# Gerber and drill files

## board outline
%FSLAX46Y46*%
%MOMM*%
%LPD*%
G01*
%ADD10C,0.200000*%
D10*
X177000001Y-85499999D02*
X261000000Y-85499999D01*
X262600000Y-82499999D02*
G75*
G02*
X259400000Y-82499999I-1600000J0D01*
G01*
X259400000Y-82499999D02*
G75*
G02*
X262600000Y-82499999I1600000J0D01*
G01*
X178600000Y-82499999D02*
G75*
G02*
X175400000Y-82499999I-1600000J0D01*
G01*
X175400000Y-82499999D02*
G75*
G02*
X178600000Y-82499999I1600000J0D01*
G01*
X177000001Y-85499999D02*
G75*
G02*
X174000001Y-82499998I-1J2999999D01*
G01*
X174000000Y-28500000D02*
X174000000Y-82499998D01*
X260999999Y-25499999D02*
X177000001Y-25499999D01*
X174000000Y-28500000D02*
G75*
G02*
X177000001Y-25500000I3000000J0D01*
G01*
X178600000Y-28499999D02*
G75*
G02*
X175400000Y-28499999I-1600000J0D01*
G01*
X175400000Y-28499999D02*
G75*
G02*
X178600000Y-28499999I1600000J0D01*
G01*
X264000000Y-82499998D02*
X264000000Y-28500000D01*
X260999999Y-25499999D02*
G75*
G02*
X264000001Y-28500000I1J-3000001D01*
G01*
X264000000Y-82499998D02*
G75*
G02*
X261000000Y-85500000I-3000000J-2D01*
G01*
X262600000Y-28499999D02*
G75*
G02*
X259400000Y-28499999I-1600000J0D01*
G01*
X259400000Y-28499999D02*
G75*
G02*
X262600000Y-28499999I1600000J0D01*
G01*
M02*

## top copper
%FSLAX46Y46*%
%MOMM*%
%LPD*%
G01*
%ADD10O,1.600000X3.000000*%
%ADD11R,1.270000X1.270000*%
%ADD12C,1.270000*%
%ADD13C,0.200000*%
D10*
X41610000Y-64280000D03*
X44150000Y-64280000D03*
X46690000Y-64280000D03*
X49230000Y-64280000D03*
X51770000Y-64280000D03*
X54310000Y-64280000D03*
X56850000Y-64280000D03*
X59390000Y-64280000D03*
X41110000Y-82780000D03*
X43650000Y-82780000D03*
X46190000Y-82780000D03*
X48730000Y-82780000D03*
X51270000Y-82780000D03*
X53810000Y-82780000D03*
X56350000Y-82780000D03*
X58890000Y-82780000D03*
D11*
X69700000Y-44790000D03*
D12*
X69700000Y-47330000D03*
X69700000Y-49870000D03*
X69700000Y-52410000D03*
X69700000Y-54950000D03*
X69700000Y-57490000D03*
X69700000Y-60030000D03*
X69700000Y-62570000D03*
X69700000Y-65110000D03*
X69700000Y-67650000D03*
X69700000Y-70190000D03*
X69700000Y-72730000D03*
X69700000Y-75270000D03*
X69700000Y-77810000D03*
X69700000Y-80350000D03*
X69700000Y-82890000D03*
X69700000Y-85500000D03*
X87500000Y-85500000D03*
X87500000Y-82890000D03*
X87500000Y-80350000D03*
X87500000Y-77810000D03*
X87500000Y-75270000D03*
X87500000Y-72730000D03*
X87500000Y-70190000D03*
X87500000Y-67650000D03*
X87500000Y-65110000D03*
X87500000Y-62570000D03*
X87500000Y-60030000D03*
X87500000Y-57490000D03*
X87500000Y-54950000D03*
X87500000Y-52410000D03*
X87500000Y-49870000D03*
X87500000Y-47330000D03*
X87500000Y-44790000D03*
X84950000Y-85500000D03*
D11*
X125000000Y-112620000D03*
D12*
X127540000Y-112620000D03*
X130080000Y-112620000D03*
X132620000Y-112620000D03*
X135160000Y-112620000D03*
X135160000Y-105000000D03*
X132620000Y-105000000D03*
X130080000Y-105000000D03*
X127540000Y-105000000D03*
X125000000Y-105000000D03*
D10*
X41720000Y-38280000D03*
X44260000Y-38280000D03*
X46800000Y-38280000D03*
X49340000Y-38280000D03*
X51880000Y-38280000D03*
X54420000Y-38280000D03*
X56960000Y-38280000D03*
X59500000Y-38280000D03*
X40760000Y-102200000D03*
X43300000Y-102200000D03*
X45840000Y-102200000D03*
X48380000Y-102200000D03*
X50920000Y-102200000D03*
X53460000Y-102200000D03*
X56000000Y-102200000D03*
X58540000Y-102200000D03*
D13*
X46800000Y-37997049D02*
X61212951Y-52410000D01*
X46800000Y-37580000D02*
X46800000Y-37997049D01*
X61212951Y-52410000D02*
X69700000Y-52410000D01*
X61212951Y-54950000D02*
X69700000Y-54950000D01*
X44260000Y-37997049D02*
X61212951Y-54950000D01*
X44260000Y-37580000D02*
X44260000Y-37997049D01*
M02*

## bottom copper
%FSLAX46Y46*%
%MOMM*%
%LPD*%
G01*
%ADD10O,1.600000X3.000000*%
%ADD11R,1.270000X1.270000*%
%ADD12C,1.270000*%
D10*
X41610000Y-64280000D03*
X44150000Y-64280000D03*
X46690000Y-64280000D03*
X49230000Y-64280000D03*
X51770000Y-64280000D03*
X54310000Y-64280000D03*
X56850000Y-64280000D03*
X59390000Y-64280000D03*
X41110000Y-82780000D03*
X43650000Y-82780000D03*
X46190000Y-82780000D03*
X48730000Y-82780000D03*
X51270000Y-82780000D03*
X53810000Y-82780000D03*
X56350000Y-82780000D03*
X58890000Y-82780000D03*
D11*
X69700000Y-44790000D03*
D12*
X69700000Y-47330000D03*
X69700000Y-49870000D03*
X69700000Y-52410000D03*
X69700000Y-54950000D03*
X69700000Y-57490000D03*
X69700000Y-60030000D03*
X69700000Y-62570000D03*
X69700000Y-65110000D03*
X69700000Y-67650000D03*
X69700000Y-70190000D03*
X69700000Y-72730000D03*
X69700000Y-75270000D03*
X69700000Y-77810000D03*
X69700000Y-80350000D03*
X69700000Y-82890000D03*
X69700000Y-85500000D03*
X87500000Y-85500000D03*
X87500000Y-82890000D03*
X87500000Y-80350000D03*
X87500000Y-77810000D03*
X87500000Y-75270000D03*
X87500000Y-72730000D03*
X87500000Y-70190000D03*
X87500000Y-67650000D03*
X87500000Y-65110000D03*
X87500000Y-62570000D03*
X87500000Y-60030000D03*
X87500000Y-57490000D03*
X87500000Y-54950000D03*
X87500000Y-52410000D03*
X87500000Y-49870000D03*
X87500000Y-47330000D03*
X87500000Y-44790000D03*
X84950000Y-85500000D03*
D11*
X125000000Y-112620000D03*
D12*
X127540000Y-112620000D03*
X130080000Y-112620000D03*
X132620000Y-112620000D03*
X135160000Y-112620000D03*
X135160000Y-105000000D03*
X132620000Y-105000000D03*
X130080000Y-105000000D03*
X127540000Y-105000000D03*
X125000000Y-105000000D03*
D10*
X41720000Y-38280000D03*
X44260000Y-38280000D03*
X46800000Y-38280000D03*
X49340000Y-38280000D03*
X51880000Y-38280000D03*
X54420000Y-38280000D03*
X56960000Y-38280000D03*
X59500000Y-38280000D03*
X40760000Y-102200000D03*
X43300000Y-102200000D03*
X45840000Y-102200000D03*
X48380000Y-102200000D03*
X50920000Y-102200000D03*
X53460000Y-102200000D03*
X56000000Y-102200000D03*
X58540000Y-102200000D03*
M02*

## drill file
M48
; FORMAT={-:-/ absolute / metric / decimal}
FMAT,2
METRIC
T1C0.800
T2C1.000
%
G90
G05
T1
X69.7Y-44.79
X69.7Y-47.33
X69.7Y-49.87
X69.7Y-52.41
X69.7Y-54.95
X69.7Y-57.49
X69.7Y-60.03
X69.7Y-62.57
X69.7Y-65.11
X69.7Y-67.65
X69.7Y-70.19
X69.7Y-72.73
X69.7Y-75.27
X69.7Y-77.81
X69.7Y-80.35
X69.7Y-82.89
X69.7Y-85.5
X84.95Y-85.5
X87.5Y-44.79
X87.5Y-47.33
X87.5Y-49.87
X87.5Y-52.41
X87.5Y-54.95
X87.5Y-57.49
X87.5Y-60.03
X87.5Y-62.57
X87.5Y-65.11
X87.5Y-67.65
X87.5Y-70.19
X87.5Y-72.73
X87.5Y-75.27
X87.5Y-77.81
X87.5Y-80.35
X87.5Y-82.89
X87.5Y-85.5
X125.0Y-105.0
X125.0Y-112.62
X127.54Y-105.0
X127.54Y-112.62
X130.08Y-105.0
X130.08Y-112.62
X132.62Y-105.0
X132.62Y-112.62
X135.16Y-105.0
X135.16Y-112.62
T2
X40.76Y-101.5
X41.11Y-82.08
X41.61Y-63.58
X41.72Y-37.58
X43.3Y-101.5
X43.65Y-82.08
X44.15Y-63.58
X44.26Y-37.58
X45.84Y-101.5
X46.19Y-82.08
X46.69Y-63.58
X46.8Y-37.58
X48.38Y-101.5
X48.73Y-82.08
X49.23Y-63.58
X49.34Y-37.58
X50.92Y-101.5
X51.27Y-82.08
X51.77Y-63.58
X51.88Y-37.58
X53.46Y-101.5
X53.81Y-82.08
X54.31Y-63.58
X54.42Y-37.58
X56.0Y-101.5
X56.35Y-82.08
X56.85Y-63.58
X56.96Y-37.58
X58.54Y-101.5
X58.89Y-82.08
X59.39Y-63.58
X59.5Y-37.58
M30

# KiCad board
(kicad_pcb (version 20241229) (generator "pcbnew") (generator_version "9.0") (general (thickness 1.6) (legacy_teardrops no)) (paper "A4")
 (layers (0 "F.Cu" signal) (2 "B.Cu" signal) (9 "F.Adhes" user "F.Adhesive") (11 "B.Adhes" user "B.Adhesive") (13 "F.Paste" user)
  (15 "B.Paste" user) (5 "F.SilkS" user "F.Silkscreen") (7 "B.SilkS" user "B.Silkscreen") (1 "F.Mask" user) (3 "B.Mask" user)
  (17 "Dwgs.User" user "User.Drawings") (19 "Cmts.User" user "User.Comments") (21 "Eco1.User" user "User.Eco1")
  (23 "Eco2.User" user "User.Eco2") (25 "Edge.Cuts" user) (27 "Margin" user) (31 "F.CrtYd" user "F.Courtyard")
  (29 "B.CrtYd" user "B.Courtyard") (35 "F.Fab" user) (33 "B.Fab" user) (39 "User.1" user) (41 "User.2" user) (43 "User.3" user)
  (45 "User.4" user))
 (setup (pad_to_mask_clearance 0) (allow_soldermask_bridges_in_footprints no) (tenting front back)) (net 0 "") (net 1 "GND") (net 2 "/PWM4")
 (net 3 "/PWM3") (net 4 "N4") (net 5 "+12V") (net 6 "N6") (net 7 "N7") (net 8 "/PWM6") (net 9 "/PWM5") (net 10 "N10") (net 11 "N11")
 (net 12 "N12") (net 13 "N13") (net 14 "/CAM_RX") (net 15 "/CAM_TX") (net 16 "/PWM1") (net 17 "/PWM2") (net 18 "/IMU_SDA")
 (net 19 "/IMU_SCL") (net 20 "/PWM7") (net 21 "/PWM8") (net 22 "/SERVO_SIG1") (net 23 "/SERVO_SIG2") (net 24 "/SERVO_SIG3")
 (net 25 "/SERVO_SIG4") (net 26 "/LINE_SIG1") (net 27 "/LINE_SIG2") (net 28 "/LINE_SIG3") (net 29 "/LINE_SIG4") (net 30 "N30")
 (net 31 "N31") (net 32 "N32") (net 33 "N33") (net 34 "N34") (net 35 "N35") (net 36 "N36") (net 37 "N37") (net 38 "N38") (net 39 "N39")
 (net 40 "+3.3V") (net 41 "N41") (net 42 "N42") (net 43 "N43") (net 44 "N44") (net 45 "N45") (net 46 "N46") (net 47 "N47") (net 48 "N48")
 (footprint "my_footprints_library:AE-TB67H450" (layer "F.Cu") (at 50.5 61.5)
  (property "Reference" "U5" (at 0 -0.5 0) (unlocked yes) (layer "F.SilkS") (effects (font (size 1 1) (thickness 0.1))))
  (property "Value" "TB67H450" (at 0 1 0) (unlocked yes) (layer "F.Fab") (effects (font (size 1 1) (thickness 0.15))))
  (pad "1" thru_hole oval (at -8.89 2.08) (size 1.6 3) (drill 1 (offset 0 0.7)) (layers "*.Cu" "*.Mask") (remove_unused_layers no)
   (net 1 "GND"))
  (pad "2" thru_hole oval (at -6.35 2.08) (size 1.6 3) (drill 1 (offset 0 0.7)) (layers "*.Cu" "*.Mask") (remove_unused_layers no)
   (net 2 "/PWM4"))
  (pad "3" thru_hole oval (at -3.81 2.08) (size 1.6 3) (drill 1 (offset 0 0.7)) (layers "*.Cu" "*.Mask") (remove_unused_layers no)
   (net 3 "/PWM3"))
  (pad "4" thru_hole oval (at -1.27 2.08) (size 1.6 3) (drill 1 (offset 0 0.7)) (layers "*.Cu" "*.Mask") (remove_unused_layers no)
   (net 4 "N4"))
  (pad "5" thru_hole oval (at 1.27 2.08) (size 1.6 3) (drill 1 (offset 0 0.7)) (layers "*.Cu" "*.Mask") (remove_unused_layers no)
   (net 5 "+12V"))
  (pad "6" thru_hole oval (at 3.81 2.08) (size 1.6 3) (drill 1 (offset 0 0.7)) (layers "*.Cu" "*.Mask") (remove_unused_layers no)
   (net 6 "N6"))
  (pad "7" thru_hole oval (at 6.35 2.08) (size 1.6 3) (drill 1 (offset 0 0.7)) (layers "*.Cu" "*.Mask") (remove_unused_layers no)
   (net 1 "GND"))
  (pad "8" thru_hole oval (at 8.89 2.08) (size 1.6 3) (drill 1 (offset 0 0.7)) (layers "*.Cu" "*.Mask") (remove_unused_layers no)
   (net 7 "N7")))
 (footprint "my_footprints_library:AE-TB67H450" (layer "F.Cu") (at 50 80)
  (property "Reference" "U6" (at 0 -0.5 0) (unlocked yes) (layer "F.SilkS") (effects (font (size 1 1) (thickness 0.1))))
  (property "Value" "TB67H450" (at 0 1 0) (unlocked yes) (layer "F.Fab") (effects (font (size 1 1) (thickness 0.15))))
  (pad "1" thru_hole oval (at -8.89 2.08) (size 1.6 3) (drill 1 (offset 0 0.7)) (layers "*.Cu" "*.Mask") (remove_unused_layers no)
   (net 1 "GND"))
  (pad "2" thru_hole oval (at -6.35 2.08) (size 1.6 3) (drill 1 (offset 0 0.7)) (layers "*.Cu" "*.Mask") (remove_unused_layers no)
   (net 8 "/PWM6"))
  (pad "3" thru_hole oval (at -3.81 2.08) (size 1.6 3) (drill 1 (offset 0 0.7)) (layers "*.Cu" "*.Mask") (remove_unused_layers no)
   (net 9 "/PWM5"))
  (pad "4" thru_hole oval (at -1.27 2.08) (size 1.6 3) (drill 1 (offset 0 0.7)) (layers "*.Cu" "*.Mask") (remove_unused_layers no)
   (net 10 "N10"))
  (pad "5" thru_hole oval (at 1.27 2.08) (size 1.6 3) (drill 1 (offset 0 0.7)) (layers "*.Cu" "*.Mask") (remove_unused_layers no)
   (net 5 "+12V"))
  (pad "6" thru_hole oval (at 3.81 2.08) (size 1.6 3) (drill 1 (offset 0 0.7)) (layers "*.Cu" "*.Mask") (remove_unused_layers no)
   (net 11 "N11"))
  (pad "7" thru_hole oval (at 6.35 2.08) (size 1.6 3) (drill 1 (offset 0 0.7)) (layers "*.Cu" "*.Mask") (remove_unused_layers no)
   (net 1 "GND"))
  (pad "8" thru_hole oval (at 8.89 2.08) (size 1.6 3) (drill 1 (offset 0 0.7)) (layers "*.Cu" "*.Mask") (remove_unused_layers no)
   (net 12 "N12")))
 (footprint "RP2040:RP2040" (layer "F.Cu") (at 78.6 65.11)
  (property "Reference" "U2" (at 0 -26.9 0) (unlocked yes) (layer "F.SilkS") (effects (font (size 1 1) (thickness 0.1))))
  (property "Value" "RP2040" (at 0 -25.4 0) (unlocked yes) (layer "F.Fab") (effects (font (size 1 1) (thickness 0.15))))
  (pad "1" thru_hole rect (at -8.9 -20.32) (size 1.27 1.27) (drill 0.8) (layers "*.Cu" "*.Mask") (remove_unused_layers no) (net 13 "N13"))
  (pad "2" thru_hole circle (at -8.9 -17.78) (size 1.27 1.27) (drill 0.8) (layers "*.Cu" "*.Mask") (remove_unused_layers no)
   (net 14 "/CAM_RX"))
  (pad "3" thru_hole circle (at -8.9 -15.24) (size 1.27 1.27) (drill 0.8) (layers "*.Cu" "*.Mask") (remove_unused_layers no)
   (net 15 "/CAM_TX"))
  (pad "4" thru_hole circle (at -8.9 -12.7) (size 1.27 1.27) (drill 0.8) (layers "*.Cu" "*.Mask") (remove_unused_layers no) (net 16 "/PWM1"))
  (pad "5" thru_hole circle (at -8.9 -10.16) (size 1.27 1.27) (drill 0.8) (layers "*.Cu" "*.Mask") (remove_unused_layers no)
   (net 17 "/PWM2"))
  (pad "6" thru_hole circle (at -8.9 -7.62) (size 1.27 1.27) (drill 0.8) (layers "*.Cu" "*.Mask") (remove_unused_layers no) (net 3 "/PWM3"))
  (pad "7" thru_hole circle (at -8.9 -5.08) (size 1.27 1.27) (drill 0.8) (layers "*.Cu" "*.Mask") (remove_unused_layers no) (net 2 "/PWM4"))
  (pad "8" thru_hole circle (at -8.9 -2.54) (size 1.27 1.27) (drill 0.8) (layers "*.Cu" "*.Mask") (remove_unused_layers no)
   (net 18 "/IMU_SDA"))
  (pad "9" thru_hole circle (at -8.9 0) (size 1.27 1.27) (drill 0.8) (layers "*.Cu" "*.Mask") (remove_unused_layers no) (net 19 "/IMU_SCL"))
  (pad "10" thru_hole circle (at -8.9 2.54) (size 1.27 1.27) (drill 0.8) (layers "*.Cu" "*.Mask") (remove_unused_layers no) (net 9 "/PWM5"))
  (pad "11" thru_hole circle (at -8.9 5.08) (size 1.27 1.27) (drill 0.8) (layers "*.Cu" "*.Mask") (remove_unused_layers no) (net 8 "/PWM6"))
  (pad "12" thru_hole circle (at -8.9 7.62) (size 1.27 1.27) (drill 0.8) (layers "*.Cu" "*.Mask") (remove_unused_layers no) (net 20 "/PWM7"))
  (pad "13" thru_hole circle (at -8.9 10.16) (size 1.27 1.27) (drill 0.8) (layers "*.Cu" "*.Mask") (remove_unused_layers no)
   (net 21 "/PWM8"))
  (pad "14" thru_hole circle (at -8.9 12.7) (size 1.27 1.27) (drill 0.8) (layers "*.Cu" "*.Mask") (remove_unused_layers no)
   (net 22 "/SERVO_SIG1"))
  (pad "15" thru_hole circle (at -8.9 15.24) (size 1.27 1.27) (drill 0.8) (layers "*.Cu" "*.Mask") (remove_unused_layers no)
   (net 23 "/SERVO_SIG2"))
  (pad "16" thru_hole circle (at -8.9 17.78) (size 1.27 1.27) (drill 0.8) (layers "*.Cu" "*.Mask") (remove_unused_layers no)
   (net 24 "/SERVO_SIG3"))
  (pad "17" thru_hole circle (at -8.9 20.39) (size 1.27 1.27) (drill 0.8) (layers "*.Cu" "*.Mask") (remove_unused_layers no)
   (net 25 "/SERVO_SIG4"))
  (pad "18" thru_hole circle (at 8.9 20.39) (size 1.27 1.27) (drill 0.8) (layers "*.Cu" "*.Mask") (remove_unused_layers no) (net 1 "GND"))
  (pad "19" thru_hole circle (at 8.9 17.78) (size 1.27 1.27) (drill 0.8) (layers "*.Cu" "*.Mask") (remove_unused_layers no)
   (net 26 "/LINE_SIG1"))
  (pad "20" thru_hole circle (at 8.9 15.24) (size 1.27 1.27) (drill 0.8) (layers "*.Cu" "*.Mask") (remove_unused_layers no)
   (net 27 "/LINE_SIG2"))
  (pad "21" thru_hole circle (at 8.9 12.7) (size 1.27 1.27) (drill 0.8) (layers "*.Cu" "*.Mask") (remove_unused_layers no)
   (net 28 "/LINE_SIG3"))
  (pad "22" thru_hole circle (at 8.9 10.16) (size 1.27 1.27) (drill 0.8) (layers "*.Cu" "*.Mask") (remove_unused_layers no)
   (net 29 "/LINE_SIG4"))
  (pad "23" thru_hole circle (at 8.9 7.62) (size 1.27 1.27) (drill 0.8) (layers "*.Cu" "*.Mask") (remove_unused_layers no) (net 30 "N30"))
  (pad "24" thru_hole circle (at 8.9 5.08) (size 1.27 1.27) (drill 0.8) (layers "*.Cu" "*.Mask") (remove_unused_layers no) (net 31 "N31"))
  (pad "25" thru_hole circle (at 8.9 2.54) (size 1.27 1.27) (drill 0.8) (layers "*.Cu" "*.Mask") (remove_unused_layers no) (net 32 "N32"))
  (pad "26" thru_hole circle (at 8.9 0) (size 1.27 1.27) (drill 0.8) (layers "*.Cu" "*.Mask") (remove_unused_layers no) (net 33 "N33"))
  (pad "27" thru_hole circle (at 8.9 -2.54) (size 1.27 1.27) (drill 0.8) (layers "*.Cu" "*.Mask") (remove_unused_layers no) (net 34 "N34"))
  (pad "28" thru_hole circle (at 8.9 -5.08) (size 1.27 1.27) (drill 0.8) (layers "*.Cu" "*.Mask") (remove_unused_layers no) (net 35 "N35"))
  (pad "29" thru_hole circle (at 8.9 -7.62) (size 1.27 1.27) (drill 0.8) (layers "*.Cu" "*.Mask") (remove_unused_layers no) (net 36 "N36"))
  (pad "30" thru_hole circle (at 8.9 -10.16) (size 1.27 1.27) (drill 0.8) (layers "*.Cu" "*.Mask") (remove_unused_layers no) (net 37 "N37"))
  (pad "31" thru_hole circle (at 8.9 -12.7) (size 1.27 1.27) (drill 0.8) (layers "*.Cu" "*.Mask") (remove_unused_layers no) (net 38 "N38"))
  (pad "32" thru_hole circle (at 8.9 -15.24) (size 1.27 1.27) (drill 0.8) (layers "*.Cu" "*.Mask") (remove_unused_layers no) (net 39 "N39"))
  (pad "33" thru_hole circle (at 8.9 -17.78) (size 1.27 1.27) (drill 0.8) (layers "*.Cu" "*.Mask") (remove_unused_layers no) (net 1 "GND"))
  (pad "34" thru_hole circle (at 8.9 -20.32) (size 1.27 1.27) (drill 0.8) (layers "*.Cu" "*.Mask") (remove_unused_layers no)
   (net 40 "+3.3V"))
  (pad "35" thru_hole circle (at 6.35 20.39) (size 1.27 1.27) (drill 0.8) (layers "*.Cu" "*.Mask") (remove_unused_layers no) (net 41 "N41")))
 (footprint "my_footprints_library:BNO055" (layer "F.Cu") (at 130.08 108.81)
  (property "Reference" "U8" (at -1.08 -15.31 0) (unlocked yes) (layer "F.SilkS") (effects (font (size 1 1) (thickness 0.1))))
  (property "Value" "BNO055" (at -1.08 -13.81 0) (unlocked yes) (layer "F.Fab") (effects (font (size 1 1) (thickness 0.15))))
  (pad "1" thru_hole rect (at -5.08 3.81) (size 1.27 1.27) (drill 0.8) (layers "*.Cu" "*.Mask") (remove_unused_layers no) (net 40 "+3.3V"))
  (pad "2" thru_hole circle (at -2.54 3.81) (size 1.27 1.27) (drill 0.8) (layers "*.Cu" "*.Mask") (remove_unused_layers no) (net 40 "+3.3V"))
  (pad "3" thru_hole circle (at 0 3.81) (size 1.27 1.27) (drill 0.8) (layers "*.Cu" "*.Mask") (remove_unused_layers no) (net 19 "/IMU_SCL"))
  (pad "4" thru_hole circle (at 2.54 3.81) (size 1.27 1.27) (drill 0.8) (layers "*.Cu" "*.Mask") (remove_unused_layers no)
   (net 18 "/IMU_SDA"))
  (pad "5" thru_hole circle (at 5.08 3.81) (size 1.27 1.27) (drill 0.8) (layers "*.Cu" "*.Mask") (remove_unused_layers no) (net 1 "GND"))
  (pad "6" thru_hole circle (at 5.08 -3.81) (size 1.27 1.27) (drill 0.8) (layers "*.Cu" "*.Mask") (remove_unused_layers no) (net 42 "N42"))
  (pad "7" thru_hole circle (at 2.54 -3.81) (size 1.27 1.27) (drill 0.8) (layers "*.Cu" "*.Mask") (remove_unused_layers no) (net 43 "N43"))
  (pad "8" thru_hole circle (at 0 -3.81) (size 1.27 1.27) (drill 0.8) (layers "*.Cu" "*.Mask") (remove_unused_layers no) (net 1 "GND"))
  (pad "9" thru_hole circle (at -2.54 -3.81) (size 1.27 1.27) (drill 0.8) (layers "*.Cu" "*.Mask") (remove_unused_layers no) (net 1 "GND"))
  (pad "10" thru_hole circle (at -5.08 -3.81) (size 1.27 1.27) (drill 0.8) (layers "*.Cu" "*.Mask") (remove_unused_layers no) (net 1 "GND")))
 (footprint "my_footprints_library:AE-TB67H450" (layer "F.Cu") (at 50.61 35.5)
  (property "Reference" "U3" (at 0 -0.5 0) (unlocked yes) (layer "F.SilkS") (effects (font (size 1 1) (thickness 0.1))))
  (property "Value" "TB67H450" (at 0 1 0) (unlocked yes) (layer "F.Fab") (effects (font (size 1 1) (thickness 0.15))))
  (pad "1" thru_hole oval (at -8.89 2.08) (size 1.6 3) (drill 1 (offset 0 0.7)) (layers "*.Cu" "*.Mask") (remove_unused_layers no)
   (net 1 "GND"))
  (pad "2" thru_hole oval (at -6.35 2.08) (size 1.6 3) (drill 1 (offset 0 0.7)) (layers "*.Cu" "*.Mask") (remove_unused_layers no)
   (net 17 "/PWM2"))
  (pad "3" thru_hole oval (at -3.81 2.08) (size 1.6 3) (drill 1 (offset 0 0.7)) (layers "*.Cu" "*.Mask") (remove_unused_layers no)
   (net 16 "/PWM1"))
  (pad "4" thru_hole oval (at -1.27 2.08) (size 1.6 3) (drill 1 (offset 0 0.7)) (layers "*.Cu" "*.Mask") (remove_unused_layers no)
   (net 40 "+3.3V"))
  (pad "5" thru_hole oval (at 1.27 2.08) (size 1.6 3) (drill 1 (offset 0 0.7)) (layers "*.Cu" "*.Mask") (remove_unused_layers no)
   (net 5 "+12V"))
  (pad "6" thru_hole oval (at 3.81 2.08) (size 1.6 3) (drill 1 (offset 0 0.7)) (layers "*.Cu" "*.Mask") (remove_unused_layers no)
   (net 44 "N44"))
  (pad "7" thru_hole oval (at 6.35 2.08) (size 1.6 3) (drill 1 (offset 0 0.7)) (layers "*.Cu" "*.Mask") (remove_unused_layers no)
   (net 1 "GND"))
  (pad "8" thru_hole oval (at 8.89 2.08) (size 1.6 3) (drill 1 (offset 0 0.7)) (layers "*.Cu" "*.Mask") (remove_unused_layers no)
   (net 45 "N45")))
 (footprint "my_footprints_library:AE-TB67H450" (layer "F.Cu") (at 49.65 99.42)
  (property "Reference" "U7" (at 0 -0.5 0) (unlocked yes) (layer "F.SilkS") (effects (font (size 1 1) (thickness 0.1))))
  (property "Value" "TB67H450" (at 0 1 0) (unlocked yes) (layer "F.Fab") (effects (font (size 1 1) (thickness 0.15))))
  (pad "1" thru_hole oval (at -8.89 2.08) (size 1.6 3) (drill 1 (offset 0 0.7)) (layers "*.Cu" "*.Mask") (remove_unused_layers no)
   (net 1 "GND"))
  (pad "2" thru_hole oval (at -6.35 2.08) (size 1.6 3) (drill 1 (offset 0 0.7)) (layers "*.Cu" "*.Mask") (remove_unused_layers no)
   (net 21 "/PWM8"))
  (pad "3" thru_hole oval (at -3.81 2.08) (size 1.6 3) (drill 1 (offset 0 0.7)) (layers "*.Cu" "*.Mask") (remove_unused_layers no)
   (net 20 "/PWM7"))
  (pad "4" thru_hole oval (at -1.27 2.08) (size 1.6 3) (drill 1 (offset 0 0.7)) (layers "*.Cu" "*.Mask") (remove_unused_layers no)
   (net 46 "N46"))
  (pad "5" thru_hole oval (at 1.27 2.08) (size 1.6 3) (drill 1 (offset 0 0.7)) (layers "*.Cu" "*.Mask") (remove_unused_layers no)
   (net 5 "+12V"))
  (pad "6" thru_hole oval (at 3.81 2.08) (size 1.6 3) (drill 1 (offset 0 0.7)) (layers "*.Cu" "*.Mask") (remove_unused_layers no)
   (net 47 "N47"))
  (pad "7" thru_hole oval (at 6.35 2.08) (size 1.6 3) (drill 1 (offset 0 0.7)) (layers "*.Cu" "*.Mask") (remove_unused_layers no)
   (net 1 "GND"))
  (pad "8" thru_hole oval (at 8.89 2.08) (size 1.6 3) (drill 1 (offset 0 0.7)) (layers "*.Cu" "*.Mask") (remove_unused_layers no)
   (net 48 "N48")))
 (gr_line (start 177.000001 85.499999) (end 261 85.499999) (stroke (width 0.2) (type default)) (layer "Edge.Cuts"))
 (gr_circle (center 261 82.499999) (end 262.6 82.499999) (stroke (width 0.2) (type default)) (fill no) (layer "Edge.Cuts"))
 (gr_circle (center 177 82.499999) (end 178.6 82.499999) (stroke (width 0.2) (type default)) (fill no) (layer "Edge.Cuts"))
 (gr_arc (start 177.000001 85.499999) (mid 174.87868 84.621319) (end 174 82.499998) (stroke (width 0.2) (type default)) (layer "Edge.Cuts"))
 (gr_line (start 174 28.5) (end 174 82.499998) (stroke (width 0.2) (type default)) (layer "Edge.Cuts"))
 (gr_line (start 260.999999 25.499999) (end 177.000001 25.499999) (stroke (width 0.2) (type default)) (layer "Edge.Cuts"))
 (gr_arc (start 174 28.5) (mid 174.87868 26.378679) (end 177.000001 25.499999) (stroke (width 0.2) (type default)) (layer "Edge.Cuts"))
 (gr_circle (center 177 28.499999) (end 178.6 28.499999) (stroke (width 0.2) (type default)) (fill no) (layer "Edge.Cuts"))
 (gr_line (start 264 82.499998) (end 264 28.5) (stroke (width 0.2) (type default)) (layer "Edge.Cuts"))
 (gr_arc (start 260.999999 25.499999) (mid 263.12132 26.378679) (end 264 28.5) (stroke (width 0.2) (type default)) (layer "Edge.Cuts"))
 (gr_arc (start 264 82.499998) (mid 263.12132 84.621319) (end 261 85.499999) (stroke (width 0.2) (type default)) (layer "Edge.Cuts"))
 (gr_circle (center 261 28.499999) (end 262.6 28.499999) (stroke (width 0.2) (type default)) (fill no) (layer "Edge.Cuts"))
 (segment (start 46.8 37.997049) (end 61.212951 52.41) (width 0.2) (layer "F.Cu") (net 16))
 (segment (start 46.8 37.58) (end 46.8 37.997049) (width 0.2) (layer "F.Cu") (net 16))
 (segment (start 61.212951 52.41) (end 69.7 52.41) (width 0.2) (layer "F.Cu") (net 16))
 (segment (start 61.212951 54.95) (end 69.7 54.95) (width 0.2) (layer "F.Cu") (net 17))
 (segment (start 44.26 37.997049) (end 61.212951 54.95) (width 0.2) (layer "F.Cu") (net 17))
 (segment (start 44.26 37.58) (end 44.26 37.997049) (width 0.2) (layer "F.Cu") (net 17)))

